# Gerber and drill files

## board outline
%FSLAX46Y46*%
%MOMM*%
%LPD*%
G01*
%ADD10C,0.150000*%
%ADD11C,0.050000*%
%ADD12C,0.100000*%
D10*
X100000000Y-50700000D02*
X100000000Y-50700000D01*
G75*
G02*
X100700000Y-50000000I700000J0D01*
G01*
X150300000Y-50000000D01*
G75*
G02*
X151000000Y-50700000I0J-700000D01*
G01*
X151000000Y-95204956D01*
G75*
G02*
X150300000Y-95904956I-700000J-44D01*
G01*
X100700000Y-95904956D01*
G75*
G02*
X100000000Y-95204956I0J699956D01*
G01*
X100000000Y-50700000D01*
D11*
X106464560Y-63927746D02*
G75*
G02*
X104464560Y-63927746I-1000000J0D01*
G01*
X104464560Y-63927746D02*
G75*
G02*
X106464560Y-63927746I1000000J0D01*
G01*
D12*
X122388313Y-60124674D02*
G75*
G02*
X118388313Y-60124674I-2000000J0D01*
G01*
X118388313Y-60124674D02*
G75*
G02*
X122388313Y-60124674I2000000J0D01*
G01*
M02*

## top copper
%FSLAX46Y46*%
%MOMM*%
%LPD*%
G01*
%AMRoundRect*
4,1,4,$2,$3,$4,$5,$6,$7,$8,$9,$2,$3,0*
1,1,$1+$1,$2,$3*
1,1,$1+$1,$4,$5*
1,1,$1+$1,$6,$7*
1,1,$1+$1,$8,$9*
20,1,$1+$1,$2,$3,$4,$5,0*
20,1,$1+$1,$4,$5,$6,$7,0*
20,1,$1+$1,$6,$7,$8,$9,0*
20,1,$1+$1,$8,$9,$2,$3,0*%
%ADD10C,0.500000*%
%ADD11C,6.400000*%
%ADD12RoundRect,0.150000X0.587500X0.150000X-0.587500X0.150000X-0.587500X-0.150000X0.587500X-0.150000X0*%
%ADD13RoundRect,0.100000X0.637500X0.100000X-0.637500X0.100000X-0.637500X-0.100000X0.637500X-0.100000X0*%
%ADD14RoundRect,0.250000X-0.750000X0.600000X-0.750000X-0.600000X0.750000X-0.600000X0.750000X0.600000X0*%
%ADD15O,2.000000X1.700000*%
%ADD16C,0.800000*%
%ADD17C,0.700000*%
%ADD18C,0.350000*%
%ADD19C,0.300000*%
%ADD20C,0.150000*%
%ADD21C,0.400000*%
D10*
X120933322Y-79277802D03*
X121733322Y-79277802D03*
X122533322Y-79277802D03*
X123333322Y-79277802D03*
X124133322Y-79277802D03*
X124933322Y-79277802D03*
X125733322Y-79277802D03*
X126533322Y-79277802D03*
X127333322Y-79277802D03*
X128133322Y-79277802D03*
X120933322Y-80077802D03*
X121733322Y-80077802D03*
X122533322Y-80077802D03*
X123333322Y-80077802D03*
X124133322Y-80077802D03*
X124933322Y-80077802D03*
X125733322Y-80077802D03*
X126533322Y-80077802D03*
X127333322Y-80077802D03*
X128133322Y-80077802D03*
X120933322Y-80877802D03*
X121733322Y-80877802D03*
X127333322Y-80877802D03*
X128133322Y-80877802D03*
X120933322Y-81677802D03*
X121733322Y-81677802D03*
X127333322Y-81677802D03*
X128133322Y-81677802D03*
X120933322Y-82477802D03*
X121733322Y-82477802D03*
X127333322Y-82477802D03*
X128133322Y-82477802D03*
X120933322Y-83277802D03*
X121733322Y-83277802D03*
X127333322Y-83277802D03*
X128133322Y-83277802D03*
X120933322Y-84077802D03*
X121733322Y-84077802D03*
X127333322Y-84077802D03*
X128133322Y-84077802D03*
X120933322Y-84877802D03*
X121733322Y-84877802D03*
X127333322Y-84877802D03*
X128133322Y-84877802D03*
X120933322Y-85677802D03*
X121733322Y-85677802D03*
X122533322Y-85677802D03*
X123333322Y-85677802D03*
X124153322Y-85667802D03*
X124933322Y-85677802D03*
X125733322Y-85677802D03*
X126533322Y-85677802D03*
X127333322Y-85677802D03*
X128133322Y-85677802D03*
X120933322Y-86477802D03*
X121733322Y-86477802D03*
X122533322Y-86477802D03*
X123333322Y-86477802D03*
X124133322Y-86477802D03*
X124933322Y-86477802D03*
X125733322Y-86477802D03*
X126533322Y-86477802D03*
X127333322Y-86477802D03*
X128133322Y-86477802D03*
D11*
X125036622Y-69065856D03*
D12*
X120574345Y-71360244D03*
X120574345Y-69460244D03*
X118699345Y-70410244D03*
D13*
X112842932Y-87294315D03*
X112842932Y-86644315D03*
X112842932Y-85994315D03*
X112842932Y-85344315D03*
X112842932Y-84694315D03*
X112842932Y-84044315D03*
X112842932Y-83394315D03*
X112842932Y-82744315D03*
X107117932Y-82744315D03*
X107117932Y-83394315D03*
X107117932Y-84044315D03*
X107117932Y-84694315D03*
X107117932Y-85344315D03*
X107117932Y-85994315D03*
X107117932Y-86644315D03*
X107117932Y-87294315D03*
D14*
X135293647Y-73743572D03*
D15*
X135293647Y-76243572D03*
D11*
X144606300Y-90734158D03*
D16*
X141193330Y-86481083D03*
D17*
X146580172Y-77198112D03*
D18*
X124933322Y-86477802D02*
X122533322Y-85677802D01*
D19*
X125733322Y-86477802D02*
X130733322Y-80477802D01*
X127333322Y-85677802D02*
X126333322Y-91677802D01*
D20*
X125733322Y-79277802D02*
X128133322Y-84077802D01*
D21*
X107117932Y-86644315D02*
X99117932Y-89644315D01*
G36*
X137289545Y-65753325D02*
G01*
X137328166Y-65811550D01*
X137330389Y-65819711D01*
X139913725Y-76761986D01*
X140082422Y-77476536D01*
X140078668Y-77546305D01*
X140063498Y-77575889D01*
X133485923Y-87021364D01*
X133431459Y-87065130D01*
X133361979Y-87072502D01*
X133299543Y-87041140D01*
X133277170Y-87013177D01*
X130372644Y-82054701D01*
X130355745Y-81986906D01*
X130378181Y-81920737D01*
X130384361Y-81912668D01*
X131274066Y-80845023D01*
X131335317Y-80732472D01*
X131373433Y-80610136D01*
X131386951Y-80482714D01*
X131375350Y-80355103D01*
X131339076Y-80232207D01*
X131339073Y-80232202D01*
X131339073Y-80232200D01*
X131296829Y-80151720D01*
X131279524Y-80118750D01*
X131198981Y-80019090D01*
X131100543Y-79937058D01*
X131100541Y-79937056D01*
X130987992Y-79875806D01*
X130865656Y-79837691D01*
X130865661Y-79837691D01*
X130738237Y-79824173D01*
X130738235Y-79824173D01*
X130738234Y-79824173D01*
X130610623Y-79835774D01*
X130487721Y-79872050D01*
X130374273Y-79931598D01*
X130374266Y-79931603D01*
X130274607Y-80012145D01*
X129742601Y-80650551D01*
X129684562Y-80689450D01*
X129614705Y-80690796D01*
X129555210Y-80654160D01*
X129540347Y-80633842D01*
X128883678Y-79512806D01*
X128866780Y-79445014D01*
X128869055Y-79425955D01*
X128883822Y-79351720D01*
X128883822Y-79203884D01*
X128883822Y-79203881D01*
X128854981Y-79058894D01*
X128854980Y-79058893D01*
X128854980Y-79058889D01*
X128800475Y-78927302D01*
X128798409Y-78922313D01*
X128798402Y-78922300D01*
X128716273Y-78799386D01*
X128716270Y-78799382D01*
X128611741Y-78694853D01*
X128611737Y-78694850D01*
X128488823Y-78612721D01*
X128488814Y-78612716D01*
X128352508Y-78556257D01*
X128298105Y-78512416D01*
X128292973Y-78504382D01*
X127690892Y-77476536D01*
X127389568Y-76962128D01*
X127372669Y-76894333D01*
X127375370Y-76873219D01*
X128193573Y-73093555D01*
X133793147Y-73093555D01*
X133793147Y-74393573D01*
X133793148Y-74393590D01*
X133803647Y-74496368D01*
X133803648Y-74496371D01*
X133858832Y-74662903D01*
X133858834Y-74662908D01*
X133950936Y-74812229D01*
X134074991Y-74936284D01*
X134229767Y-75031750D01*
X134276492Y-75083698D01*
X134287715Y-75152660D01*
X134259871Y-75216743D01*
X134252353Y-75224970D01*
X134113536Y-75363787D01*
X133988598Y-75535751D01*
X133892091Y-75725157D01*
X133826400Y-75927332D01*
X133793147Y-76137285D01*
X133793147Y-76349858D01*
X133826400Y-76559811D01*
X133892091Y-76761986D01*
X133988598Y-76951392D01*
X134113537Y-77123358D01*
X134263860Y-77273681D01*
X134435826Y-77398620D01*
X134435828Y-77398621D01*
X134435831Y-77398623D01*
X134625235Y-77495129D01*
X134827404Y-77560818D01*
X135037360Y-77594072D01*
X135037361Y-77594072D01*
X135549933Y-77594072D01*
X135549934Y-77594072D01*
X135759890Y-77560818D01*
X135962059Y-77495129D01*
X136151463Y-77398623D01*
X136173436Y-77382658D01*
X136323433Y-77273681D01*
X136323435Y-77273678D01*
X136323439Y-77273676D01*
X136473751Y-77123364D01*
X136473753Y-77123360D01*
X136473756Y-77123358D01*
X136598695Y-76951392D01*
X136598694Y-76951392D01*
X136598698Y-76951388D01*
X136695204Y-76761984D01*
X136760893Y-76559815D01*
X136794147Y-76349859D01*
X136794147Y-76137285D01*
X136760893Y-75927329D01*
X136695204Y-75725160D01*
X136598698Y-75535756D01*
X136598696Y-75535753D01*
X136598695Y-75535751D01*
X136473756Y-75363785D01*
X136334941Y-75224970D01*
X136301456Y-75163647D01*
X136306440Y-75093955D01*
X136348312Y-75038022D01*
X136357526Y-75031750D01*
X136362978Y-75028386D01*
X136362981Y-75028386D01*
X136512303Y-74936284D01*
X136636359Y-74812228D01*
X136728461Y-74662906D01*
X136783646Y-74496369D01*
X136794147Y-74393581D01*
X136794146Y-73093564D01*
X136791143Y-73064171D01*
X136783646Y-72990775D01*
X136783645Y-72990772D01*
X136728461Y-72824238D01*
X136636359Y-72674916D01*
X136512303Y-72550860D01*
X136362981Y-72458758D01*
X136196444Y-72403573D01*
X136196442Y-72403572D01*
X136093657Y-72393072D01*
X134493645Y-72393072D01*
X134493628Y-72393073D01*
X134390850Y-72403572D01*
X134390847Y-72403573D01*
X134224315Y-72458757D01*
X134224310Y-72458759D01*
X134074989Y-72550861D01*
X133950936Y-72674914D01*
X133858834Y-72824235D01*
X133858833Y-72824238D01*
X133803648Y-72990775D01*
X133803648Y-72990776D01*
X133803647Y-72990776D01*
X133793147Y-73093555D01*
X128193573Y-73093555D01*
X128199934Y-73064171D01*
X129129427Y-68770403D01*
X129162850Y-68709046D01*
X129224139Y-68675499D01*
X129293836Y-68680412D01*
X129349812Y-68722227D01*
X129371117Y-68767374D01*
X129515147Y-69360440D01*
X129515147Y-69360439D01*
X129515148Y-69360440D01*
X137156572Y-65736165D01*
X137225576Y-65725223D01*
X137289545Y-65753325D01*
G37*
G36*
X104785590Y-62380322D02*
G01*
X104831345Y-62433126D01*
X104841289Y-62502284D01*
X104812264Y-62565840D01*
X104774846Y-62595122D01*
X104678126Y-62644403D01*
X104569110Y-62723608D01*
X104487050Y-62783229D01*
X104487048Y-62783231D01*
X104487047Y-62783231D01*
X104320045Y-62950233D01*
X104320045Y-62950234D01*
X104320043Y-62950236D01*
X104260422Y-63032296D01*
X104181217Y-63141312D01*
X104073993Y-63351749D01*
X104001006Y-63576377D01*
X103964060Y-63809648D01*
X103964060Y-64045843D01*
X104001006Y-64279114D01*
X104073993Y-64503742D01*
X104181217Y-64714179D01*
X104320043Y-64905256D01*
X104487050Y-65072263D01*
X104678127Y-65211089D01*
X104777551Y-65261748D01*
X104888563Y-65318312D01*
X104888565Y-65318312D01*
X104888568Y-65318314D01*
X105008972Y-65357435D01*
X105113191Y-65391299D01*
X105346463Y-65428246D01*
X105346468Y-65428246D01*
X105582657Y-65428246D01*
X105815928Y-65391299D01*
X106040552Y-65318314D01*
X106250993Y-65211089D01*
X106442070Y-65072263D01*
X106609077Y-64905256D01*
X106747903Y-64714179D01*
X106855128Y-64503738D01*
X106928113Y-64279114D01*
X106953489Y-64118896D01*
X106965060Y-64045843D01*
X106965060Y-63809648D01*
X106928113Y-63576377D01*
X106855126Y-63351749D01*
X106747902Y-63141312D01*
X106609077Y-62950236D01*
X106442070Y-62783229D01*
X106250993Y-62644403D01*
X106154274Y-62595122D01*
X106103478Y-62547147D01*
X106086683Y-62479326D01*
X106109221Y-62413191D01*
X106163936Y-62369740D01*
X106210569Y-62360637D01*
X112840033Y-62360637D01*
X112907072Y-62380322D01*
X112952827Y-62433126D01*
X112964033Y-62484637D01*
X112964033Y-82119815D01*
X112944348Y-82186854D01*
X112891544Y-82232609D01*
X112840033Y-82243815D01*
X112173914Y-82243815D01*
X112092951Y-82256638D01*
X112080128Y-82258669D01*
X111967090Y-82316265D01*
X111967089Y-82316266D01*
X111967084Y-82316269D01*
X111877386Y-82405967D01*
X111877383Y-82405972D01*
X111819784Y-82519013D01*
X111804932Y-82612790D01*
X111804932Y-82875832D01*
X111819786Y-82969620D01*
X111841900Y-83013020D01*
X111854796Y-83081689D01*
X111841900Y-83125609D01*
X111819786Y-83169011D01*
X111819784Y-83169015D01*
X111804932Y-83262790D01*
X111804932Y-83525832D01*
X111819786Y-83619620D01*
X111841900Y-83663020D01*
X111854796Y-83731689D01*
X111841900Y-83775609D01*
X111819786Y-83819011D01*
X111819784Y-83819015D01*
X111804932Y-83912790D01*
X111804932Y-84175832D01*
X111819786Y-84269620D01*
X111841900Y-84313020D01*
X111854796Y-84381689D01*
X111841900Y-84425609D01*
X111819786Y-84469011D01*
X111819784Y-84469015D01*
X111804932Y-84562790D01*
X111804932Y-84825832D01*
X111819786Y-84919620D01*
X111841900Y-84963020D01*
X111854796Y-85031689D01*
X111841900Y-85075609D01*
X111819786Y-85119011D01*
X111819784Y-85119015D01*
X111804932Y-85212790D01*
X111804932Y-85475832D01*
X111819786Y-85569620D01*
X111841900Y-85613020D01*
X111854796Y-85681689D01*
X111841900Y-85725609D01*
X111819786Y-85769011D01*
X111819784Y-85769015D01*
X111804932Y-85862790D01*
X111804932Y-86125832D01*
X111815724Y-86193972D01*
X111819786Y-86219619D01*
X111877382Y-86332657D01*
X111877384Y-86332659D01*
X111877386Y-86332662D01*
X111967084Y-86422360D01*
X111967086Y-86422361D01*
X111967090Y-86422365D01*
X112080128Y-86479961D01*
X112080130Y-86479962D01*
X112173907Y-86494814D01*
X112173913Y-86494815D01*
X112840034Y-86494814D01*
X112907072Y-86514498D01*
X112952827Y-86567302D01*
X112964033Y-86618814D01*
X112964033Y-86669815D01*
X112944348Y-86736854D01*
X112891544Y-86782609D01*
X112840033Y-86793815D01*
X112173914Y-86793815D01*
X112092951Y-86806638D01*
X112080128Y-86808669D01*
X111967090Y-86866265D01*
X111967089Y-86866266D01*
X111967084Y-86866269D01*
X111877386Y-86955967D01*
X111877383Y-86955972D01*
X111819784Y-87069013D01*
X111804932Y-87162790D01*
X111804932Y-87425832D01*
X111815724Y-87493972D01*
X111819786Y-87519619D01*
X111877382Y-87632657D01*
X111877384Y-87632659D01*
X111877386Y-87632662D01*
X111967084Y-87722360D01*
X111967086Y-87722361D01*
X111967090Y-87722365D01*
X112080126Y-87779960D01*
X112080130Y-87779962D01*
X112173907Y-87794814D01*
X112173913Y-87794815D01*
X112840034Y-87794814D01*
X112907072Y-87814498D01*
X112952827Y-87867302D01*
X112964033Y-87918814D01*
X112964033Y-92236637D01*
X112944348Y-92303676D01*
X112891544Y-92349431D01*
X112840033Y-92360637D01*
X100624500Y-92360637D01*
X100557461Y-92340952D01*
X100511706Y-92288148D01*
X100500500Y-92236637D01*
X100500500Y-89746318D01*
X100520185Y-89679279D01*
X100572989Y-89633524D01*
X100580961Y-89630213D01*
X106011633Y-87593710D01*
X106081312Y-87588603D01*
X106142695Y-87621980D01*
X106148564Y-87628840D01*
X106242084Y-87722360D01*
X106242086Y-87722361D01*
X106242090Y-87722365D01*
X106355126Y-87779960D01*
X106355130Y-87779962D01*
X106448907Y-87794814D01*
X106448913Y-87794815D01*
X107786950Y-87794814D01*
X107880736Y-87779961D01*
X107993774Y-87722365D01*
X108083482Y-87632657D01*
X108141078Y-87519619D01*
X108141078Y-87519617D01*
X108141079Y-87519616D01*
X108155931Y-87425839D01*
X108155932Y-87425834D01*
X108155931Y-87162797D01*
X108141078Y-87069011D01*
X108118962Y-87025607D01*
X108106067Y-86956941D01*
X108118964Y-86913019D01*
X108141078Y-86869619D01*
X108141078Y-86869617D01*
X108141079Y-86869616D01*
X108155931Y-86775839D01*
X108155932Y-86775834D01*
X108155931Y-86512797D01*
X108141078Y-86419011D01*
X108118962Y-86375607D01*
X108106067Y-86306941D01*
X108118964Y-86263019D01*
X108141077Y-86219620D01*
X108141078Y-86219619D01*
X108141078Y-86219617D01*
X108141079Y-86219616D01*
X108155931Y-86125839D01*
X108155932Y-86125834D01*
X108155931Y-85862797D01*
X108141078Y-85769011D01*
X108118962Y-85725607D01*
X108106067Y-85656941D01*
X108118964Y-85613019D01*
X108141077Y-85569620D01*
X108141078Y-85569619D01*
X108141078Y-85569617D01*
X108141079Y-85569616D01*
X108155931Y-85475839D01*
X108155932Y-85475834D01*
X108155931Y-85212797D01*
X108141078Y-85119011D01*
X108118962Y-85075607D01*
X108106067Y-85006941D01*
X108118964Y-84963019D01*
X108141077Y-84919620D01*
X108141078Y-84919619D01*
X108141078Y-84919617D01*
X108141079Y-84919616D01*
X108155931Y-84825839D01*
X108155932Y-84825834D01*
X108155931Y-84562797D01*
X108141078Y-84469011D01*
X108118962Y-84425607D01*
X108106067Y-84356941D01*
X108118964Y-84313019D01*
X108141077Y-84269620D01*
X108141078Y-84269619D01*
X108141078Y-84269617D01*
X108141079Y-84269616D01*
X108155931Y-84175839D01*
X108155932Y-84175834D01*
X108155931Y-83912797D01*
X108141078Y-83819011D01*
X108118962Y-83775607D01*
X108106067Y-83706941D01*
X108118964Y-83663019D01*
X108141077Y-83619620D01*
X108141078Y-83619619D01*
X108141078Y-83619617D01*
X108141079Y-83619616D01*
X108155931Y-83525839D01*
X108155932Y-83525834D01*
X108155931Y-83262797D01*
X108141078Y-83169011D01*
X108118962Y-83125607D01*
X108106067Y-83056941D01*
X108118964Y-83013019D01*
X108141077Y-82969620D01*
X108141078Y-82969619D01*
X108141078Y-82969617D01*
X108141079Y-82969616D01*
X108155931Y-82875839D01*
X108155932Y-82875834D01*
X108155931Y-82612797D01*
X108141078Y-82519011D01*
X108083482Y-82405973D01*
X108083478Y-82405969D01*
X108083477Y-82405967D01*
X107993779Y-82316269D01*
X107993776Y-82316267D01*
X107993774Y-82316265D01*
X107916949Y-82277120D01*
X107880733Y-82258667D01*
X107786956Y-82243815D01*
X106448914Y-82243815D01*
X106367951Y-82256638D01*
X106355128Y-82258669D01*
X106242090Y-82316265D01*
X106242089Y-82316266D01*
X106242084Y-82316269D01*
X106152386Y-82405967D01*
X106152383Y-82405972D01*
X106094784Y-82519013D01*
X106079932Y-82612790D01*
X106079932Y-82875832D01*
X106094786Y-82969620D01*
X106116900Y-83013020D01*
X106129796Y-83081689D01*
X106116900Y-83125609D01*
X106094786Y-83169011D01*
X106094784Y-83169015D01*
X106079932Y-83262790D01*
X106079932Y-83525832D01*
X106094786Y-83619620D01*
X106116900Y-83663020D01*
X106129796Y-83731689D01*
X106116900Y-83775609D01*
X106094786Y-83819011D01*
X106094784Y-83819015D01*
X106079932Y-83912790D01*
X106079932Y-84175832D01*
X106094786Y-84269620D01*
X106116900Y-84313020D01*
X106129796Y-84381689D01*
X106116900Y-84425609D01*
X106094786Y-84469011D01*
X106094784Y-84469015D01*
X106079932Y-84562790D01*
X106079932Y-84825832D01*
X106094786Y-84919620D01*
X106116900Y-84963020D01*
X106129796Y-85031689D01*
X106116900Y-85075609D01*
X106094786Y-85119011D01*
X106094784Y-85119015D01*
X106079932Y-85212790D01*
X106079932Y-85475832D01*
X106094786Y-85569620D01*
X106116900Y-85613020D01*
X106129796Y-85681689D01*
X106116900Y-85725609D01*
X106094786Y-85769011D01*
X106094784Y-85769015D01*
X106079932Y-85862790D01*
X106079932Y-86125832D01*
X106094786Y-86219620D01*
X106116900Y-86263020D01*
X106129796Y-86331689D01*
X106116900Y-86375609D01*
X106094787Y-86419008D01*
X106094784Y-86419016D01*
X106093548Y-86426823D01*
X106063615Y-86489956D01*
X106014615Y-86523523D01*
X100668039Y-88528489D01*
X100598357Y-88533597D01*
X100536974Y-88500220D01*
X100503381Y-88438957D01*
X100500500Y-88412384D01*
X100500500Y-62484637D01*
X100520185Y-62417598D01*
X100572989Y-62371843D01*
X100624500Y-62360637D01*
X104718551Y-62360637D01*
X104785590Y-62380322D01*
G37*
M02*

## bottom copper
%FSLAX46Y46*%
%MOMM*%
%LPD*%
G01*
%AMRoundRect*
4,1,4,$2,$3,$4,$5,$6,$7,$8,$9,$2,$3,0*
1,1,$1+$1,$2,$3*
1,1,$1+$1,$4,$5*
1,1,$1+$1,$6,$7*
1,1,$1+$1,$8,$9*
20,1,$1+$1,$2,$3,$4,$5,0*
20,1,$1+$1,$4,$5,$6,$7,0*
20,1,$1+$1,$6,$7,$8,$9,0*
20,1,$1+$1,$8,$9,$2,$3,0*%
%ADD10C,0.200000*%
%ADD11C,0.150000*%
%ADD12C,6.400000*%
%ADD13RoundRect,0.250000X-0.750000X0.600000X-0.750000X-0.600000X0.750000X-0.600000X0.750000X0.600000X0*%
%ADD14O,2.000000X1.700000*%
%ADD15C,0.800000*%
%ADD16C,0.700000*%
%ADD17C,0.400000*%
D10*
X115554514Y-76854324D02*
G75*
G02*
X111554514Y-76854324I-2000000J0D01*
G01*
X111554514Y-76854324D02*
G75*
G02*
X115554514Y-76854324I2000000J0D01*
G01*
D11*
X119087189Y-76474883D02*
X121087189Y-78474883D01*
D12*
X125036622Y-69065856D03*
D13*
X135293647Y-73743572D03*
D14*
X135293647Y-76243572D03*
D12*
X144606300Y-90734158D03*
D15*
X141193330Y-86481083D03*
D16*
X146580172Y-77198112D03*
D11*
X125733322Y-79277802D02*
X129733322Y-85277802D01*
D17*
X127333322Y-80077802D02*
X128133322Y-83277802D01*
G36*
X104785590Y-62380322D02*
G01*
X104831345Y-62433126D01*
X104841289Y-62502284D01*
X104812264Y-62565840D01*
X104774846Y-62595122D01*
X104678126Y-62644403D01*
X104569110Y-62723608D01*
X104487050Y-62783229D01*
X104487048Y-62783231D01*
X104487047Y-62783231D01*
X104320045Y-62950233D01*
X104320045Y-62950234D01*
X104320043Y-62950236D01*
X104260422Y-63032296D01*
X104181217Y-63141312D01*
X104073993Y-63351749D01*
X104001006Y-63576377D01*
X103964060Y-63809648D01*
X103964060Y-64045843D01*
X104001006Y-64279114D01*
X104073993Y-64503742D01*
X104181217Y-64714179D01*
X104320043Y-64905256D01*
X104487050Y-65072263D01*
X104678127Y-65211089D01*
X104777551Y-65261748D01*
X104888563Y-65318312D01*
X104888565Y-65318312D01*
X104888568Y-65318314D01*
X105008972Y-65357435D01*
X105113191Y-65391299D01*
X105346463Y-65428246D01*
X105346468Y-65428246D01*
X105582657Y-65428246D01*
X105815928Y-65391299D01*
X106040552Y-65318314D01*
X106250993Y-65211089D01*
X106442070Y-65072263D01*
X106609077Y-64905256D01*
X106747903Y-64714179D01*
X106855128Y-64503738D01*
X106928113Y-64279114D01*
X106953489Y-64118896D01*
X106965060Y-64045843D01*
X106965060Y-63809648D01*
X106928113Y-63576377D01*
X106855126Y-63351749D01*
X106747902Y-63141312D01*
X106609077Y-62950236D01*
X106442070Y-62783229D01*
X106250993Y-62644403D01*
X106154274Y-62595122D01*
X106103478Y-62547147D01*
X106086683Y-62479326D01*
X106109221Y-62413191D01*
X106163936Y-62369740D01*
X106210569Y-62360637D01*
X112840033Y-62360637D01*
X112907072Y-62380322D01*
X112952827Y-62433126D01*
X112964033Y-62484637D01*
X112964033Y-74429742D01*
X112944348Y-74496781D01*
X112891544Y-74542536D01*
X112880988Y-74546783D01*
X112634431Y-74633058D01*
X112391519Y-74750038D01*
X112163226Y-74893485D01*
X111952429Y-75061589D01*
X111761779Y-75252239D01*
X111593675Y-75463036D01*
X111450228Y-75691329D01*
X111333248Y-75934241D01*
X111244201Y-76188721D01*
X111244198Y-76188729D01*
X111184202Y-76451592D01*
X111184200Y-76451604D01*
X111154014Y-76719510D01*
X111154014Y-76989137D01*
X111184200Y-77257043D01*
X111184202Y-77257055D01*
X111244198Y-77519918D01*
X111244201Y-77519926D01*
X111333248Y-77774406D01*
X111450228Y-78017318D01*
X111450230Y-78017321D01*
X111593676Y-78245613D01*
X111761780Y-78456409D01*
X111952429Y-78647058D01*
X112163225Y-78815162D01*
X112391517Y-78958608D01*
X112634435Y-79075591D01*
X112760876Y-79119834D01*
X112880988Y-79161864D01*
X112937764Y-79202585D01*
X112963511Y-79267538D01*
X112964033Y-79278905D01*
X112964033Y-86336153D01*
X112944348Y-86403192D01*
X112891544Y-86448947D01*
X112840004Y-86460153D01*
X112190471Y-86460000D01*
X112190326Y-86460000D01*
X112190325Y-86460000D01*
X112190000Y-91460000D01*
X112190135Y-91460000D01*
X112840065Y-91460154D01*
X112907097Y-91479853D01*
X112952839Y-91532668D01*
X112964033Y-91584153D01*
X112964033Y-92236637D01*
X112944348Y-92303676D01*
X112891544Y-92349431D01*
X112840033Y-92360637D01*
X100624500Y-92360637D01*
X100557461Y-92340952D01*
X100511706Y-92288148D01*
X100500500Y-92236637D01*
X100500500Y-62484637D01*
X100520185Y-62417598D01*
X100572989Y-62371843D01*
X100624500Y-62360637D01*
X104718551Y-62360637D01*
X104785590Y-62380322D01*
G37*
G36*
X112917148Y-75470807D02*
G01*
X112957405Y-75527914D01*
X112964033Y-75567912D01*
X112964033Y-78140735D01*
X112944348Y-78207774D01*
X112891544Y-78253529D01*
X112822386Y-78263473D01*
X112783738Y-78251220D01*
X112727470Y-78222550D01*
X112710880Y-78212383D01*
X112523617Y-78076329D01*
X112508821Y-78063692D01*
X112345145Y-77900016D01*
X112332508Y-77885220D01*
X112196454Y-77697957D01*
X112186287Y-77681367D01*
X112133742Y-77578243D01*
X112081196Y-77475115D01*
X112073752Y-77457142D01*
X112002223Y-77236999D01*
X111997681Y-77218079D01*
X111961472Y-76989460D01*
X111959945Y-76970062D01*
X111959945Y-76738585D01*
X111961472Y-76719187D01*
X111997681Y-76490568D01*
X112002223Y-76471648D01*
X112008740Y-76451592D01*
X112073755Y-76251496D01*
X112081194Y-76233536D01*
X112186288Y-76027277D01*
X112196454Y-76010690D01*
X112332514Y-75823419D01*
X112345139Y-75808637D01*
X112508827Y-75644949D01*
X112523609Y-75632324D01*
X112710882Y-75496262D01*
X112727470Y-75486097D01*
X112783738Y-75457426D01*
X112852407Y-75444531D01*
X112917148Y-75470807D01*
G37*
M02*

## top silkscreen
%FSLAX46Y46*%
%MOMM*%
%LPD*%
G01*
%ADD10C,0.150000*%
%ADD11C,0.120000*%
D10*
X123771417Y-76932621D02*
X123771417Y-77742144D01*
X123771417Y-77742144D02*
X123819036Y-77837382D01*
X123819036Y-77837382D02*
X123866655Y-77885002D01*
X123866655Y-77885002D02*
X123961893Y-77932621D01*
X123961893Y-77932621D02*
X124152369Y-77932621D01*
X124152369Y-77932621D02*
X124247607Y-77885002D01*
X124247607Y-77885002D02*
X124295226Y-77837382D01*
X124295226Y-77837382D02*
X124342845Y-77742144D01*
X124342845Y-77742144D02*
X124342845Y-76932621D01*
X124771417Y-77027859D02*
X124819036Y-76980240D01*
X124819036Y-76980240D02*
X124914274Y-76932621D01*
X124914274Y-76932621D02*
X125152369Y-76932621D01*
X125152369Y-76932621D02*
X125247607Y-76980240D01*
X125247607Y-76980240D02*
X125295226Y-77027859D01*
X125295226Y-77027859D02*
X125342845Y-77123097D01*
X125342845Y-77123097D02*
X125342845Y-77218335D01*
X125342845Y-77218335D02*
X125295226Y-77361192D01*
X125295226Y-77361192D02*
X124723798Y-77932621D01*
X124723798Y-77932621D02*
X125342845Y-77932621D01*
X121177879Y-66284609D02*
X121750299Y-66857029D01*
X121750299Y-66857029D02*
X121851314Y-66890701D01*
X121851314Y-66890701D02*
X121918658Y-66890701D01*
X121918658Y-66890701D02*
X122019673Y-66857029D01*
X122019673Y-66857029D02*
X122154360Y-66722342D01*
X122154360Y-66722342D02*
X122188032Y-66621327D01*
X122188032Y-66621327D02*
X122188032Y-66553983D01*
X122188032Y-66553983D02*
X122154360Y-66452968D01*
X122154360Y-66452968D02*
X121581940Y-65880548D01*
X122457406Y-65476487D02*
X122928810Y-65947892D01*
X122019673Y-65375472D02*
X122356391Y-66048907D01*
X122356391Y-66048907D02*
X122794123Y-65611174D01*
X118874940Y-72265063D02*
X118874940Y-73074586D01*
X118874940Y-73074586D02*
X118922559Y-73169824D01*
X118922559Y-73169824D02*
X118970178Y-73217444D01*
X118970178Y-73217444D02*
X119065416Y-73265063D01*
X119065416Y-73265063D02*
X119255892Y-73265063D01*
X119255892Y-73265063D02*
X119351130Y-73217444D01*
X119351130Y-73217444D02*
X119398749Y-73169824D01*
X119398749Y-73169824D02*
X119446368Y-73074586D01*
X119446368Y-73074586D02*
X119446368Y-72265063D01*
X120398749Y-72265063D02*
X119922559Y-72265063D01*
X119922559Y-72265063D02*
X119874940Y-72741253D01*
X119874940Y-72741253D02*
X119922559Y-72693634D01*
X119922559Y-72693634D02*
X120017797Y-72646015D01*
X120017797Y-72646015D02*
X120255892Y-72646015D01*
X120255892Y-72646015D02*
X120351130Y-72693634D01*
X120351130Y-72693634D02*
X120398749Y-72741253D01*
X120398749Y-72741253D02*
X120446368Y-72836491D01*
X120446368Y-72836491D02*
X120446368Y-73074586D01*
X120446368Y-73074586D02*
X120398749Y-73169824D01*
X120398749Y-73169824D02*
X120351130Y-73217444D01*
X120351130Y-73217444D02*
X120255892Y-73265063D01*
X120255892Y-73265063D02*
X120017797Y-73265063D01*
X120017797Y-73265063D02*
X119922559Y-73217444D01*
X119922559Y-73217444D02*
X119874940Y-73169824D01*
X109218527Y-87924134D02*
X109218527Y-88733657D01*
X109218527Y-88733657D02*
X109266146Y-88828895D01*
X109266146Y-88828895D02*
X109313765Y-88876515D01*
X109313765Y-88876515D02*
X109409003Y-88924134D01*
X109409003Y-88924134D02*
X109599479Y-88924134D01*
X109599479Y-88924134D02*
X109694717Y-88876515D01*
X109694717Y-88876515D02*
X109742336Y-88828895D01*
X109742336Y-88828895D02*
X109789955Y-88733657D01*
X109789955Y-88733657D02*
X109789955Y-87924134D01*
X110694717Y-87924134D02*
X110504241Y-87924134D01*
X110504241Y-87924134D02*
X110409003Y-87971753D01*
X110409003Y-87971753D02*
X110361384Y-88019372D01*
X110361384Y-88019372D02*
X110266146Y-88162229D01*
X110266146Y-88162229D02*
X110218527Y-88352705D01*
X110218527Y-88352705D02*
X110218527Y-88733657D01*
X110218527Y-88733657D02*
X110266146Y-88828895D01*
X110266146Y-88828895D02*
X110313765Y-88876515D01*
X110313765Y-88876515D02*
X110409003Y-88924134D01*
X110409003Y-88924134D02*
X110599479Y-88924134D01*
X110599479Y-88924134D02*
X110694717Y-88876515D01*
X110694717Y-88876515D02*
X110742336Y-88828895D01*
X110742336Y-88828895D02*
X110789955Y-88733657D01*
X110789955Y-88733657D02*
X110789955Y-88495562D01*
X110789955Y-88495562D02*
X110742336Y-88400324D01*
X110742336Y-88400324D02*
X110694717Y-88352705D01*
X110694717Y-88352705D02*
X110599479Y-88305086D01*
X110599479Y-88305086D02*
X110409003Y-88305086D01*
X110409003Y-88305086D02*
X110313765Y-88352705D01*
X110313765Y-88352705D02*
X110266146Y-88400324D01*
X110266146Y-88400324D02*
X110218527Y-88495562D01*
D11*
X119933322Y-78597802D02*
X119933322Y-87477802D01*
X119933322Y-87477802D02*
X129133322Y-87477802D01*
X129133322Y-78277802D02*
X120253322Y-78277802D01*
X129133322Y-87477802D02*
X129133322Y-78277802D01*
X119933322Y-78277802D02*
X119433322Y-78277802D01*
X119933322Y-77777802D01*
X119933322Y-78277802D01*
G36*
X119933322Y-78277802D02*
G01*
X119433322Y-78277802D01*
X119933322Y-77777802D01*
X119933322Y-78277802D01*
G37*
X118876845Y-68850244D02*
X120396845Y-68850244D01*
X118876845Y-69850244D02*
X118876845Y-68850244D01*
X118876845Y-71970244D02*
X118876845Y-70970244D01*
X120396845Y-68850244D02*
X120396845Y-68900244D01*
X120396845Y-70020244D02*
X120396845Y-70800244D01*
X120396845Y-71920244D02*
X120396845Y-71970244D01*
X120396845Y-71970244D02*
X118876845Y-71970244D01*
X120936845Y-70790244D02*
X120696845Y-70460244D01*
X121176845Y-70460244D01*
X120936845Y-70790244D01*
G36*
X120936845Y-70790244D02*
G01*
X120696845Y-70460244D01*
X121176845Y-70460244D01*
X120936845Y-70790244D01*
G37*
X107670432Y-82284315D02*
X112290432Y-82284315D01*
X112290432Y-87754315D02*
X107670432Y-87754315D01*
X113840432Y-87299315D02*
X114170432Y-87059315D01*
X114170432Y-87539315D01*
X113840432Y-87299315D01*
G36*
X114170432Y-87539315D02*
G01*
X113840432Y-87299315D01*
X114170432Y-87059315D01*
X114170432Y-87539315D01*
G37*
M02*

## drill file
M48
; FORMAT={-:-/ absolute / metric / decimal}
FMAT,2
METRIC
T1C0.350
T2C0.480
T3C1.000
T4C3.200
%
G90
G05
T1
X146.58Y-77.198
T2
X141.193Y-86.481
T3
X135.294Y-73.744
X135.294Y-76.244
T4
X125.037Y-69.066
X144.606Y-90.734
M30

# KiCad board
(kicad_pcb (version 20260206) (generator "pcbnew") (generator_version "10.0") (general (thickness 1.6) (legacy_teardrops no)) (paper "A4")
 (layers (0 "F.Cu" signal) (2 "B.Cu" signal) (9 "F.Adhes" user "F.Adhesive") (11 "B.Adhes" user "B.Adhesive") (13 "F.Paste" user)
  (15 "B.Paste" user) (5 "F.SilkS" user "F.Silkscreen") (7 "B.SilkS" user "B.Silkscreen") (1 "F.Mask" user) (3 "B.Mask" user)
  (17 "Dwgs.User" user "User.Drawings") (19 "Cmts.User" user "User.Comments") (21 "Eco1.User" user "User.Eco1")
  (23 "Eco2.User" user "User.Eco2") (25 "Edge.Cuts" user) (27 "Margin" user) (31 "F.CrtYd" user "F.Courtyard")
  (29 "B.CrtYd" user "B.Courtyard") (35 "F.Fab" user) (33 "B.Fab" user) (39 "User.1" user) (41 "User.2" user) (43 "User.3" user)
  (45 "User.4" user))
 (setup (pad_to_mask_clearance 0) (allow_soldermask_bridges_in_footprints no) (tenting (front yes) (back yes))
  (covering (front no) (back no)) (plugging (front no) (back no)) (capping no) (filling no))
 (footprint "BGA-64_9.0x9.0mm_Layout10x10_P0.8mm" (layer "F.Cu") (at 124.533322 82.877802)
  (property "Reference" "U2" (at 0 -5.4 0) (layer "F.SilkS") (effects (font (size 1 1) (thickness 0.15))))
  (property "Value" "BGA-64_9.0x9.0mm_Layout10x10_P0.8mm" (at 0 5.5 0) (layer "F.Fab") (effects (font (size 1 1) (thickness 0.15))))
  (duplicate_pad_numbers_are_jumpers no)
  (fp_line (start -4.6 -4.28) (end -4.6 4.6) (stroke (width 0.12) (type solid)) (layer "F.SilkS"))
  (fp_line (start -4.6 4.6) (end 4.6 4.6) (stroke (width 0.12) (type solid)) (layer "F.SilkS"))
  (fp_line (start 4.6 -4.6) (end -4.28 -4.6) (stroke (width 0.12) (type solid)) (layer "F.SilkS"))
  (fp_line (start 4.6 4.6) (end 4.6 -4.6) (stroke (width 0.12) (type solid)) (layer "F.SilkS"))
  (fp_poly
   (pts (xy -4.6 -4.6) (xy -5.1 -4.6) (xy -4.6 -5.1) (xy -4.6 -4.6)) (stroke (width 0.12) (type solid)) (fill yes) (layer "F.SilkS"))
  (pad "A1" smd circle (at -3.6 -3.6) (size 0.5 0.5) (layers "F.Cu" "F.Mask" "F.Paste") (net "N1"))
  (pad "A2" smd circle (at -2.8 -3.6) (size 0.5 0.5) (layers "F.Cu" "F.Mask" "F.Paste"))
  (pad "A3" smd circle (at -2 -3.6) (size 0.5 0.5) (layers "F.Cu" "F.Mask" "F.Paste") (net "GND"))
  (pad "A4" smd circle (at -1.2 -3.6) (size 0.5 0.5) (layers "F.Cu" "F.Mask" "F.Paste") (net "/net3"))
  (pad "A5" smd circle (at -0.4 -3.6) (size 0.5 0.5) (layers "F.Cu" "F.Mask" "F.Paste") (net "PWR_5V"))
  (pad "A6" smd circle (at 0.4 -3.6) (size 0.5 0.5) (layers "F.Cu" "F.Mask" "F.Paste"))
  (pad "A7" smd circle (at 1.2 -3.6) (size 0.5 0.5) (layers "F.Cu" "F.Mask" "F.Paste") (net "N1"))
  (pad "A8" smd circle (at 2 -3.6) (size 0.5 0.5) (layers "F.Cu" "F.Mask" "F.Paste") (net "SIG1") (clearance 0.1))
  (pad "A9" smd circle (at 2.8 -3.6) (size 0.5 0.5) (layers "F.Cu" "F.Mask" "F.Paste") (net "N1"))
  (pad "A10" smd circle (at 3.6 -3.6) (size 0.5 0.5) (layers "F.Cu" "F.Mask" "F.Paste") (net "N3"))
  (pad "B1" smd circle (at -3.6 -2.8) (size 0.5 0.5) (layers "F.Cu" "F.Mask" "F.Paste"))
  (pad "B2" smd circle (at -2.8 -2.8) (size 0.5 0.5) (layers "F.Cu" "F.Mask" "F.Paste") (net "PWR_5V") (clearance 0.35))
  (pad "B3" smd circle (at -2 -2.8) (size 0.5 0.5) (layers "F.Cu" "F.Mask" "F.Paste") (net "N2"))
  (pad "B4" smd circle (at -1.2 -2.8) (size 0.5 0.5) (layers "F.Cu" "F.Mask" "F.Paste"))
  (pad "B5" smd circle (at -0.4 -2.8) (size 0.5 0.5) (layers "F.Cu" "F.Mask" "F.Paste"))
  (pad "B6" smd circle (at 0.4 -2.8) (size 0.5 0.5) (layers "F.Cu" "F.Mask" "F.Paste"))
  (pad "B7" smd circle (at 1.2 -2.8) (size 0.5 0.5) (layers "F.Cu" "F.Mask" "F.Paste") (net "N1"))
  (pad "B8" smd circle (at 2 -2.8) (size 0.5 0.5) (layers "F.Cu" "F.Mask" "F.Paste"))
  (pad "B9" smd circle (at 2.8 -2.8) (size 0.5 0.5) (layers "F.Cu" "F.Mask" "F.Paste") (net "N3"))
  (pad "B10" smd circle (at 3.6 -2.8) (size 0.5 0.5) (layers "F.Cu" "F.Mask" "F.Paste") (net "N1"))
  (pad "C1" smd circle (at -3.6 -2) (size 0.5 0.5) (layers "F.Cu" "F.Mask" "F.Paste"))
  (pad "C2" smd circle (at -2.8 -2) (size 0.5 0.5) (layers "F.Cu" "F.Mask" "F.Paste") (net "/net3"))
  (pad "C9" smd circle (at 2.8 -2) (size 0.5 0.5) (layers "F.Cu" "F.Mask" "F.Paste"))
  (pad "C10" smd circle (at 3.6 -2) (size 0.5 0.5) (layers "F.Cu" "F.Mask" "F.Paste") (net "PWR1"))
  (pad "D1" smd circle (at -3.6 -1.2) (size 0.5 0.5) (layers "F.Cu" "F.Mask" "F.Paste") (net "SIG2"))
  (pad "D2" smd circle (at -2.8 -1.2) (size 0.5 0.5) (layers "F.Cu" "F.Mask" "F.Paste") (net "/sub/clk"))
  (pad "D9" smd circle (at 2.8 -1.2) (size 0.5 0.5) (layers "F.Cu" "F.Mask" "F.Paste") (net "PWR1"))
  (pad "D10" smd circle (at 3.6 -1.2) (size 0.5 0.5) (layers "F.Cu" "F.Mask" "F.Paste") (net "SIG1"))
  (pad "E1" smd circle (at -3.6 -0.4) (size 0.5 0.5) (layers "F.Cu" "F.Mask" "F.Paste") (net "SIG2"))
  (pad "E2" smd circle (at -2.8 -0.4) (size 0.5 0.5) (layers "F.Cu" "F.Mask" "F.Paste"))
  (pad "E9" smd circle (at 2.8 -0.4) (size 0.5 0.5) (layers "F.Cu" "F.Mask" "F.Paste") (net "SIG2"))
  (pad "E10" smd circle (at 3.6 -0.4) (size 0.5 0.5) (layers "F.Cu" "F.Mask" "F.Paste") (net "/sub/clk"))
  (pad "F1" smd circle (at -3.6 0.4) (size 0.5 0.5) (layers "F.Cu" "F.Mask" "F.Paste") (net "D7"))
  (pad "F2" smd circle (at -2.8 0.4) (size 0.5 0.5) (layers "F.Cu" "F.Mask" "F.Paste") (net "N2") (clearance 0.1))
  (pad "F9" smd circle (at 2.8 0.4) (size 0.5 0.5) (layers "F.Cu" "F.Mask" "F.Paste"))
  (pad "F10" smd circle (at 3.6 0.4) (size 0.5 0.5) (layers "F.Cu" "F.Mask" "F.Paste"))
  (pad "G1" smd circle (at -3.6 1.2) (size 0.5 0.5) (layers "F.Cu" "F.Mask" "F.Paste"))
  (pad "G2" smd circle (at -2.8 1.2) (size 0.5 0.5) (layers "F.Cu" "F.Mask" "F.Paste") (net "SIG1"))
  (pad "G9" smd circle (at 2.8 1.2) (size 0.5 0.5) (layers "F.Cu" "F.Mask" "F.Paste"))
  (pad "G10" smd circle (at 3.6 1.2) (size 0.5 0.5) (layers "F.Cu" "F.Mask" "F.Paste"))
  (pad "H1" smd circle (at -3.6 2) (size 0.5 0.5) (layers "F.Cu" "F.Mask" "F.Paste") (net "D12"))
  (pad "H2" smd circle (at -2.8 2) (size 0.5 0.5) (layers "F.Cu" "F.Mask" "F.Paste") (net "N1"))
  (pad "H9" smd circle (at 2.8 2) (size 0.5 0.5) (layers "F.Cu" "F.Mask" "F.Paste") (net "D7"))
  (pad "H10" smd circle (at 3.6 2) (size 0.5 0.5) (layers "F.Cu" "F.Mask" "F.Paste") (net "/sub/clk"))
  (pad "J1" smd circle (at -3.6 2.8) (size 0.5 0.5) (layers "F.Cu" "F.Mask" "F.Paste") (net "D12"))
  (pad "J2" smd circle (at -2.8 2.8) (size 0.5 0.5) (layers "F.Cu" "F.Mask" "F.Paste") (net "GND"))
  (pad "J3" smd circle (at -2 2.8) (size 0.5 0.5) (layers "F.Cu" "F.Mask" "F.Paste") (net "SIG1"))
  (pad "J4" smd circle (at -1.2 2.8) (size 0.5 0.5) (layers "F.Cu" "F.Mask" "F.Paste"))
  (pad "J5" smd circle (at -0.38 2.79) (size 0.5 0.5) (layers "F.Cu" "F.Mask" "F.Paste") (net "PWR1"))
  (pad "J6" smd circle (at 0.4 2.8) (size 0.5 0.5) (layers "F.Cu" "F.Mask" "F.Paste") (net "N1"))
  (pad "J7" smd circle (at 1.2 2.8) (size 0.5 0.5) (layers "F.Cu" "F.Mask" "F.Paste") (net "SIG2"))
  (pad "J8" smd circle (at 2 2.8) (size 0.5 0.5) (layers "F.Cu" "F.Mask" "F.Paste") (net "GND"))
  (pad "J9" smd circle (at 2.8 2.8) (size 0.5 0.5) (layers "F.Cu" "F.Mask" "F.Paste"))
  (pad "J10" smd circle (at 3.6 2.8) (size 0.5 0.5) (layers "F.Cu" "F.Mask" "F.Paste"))
  (pad "K1" smd circle (at -3.6 3.6) (size 0.5 0.5) (layers "F.Cu" "F.Mask" "F.Paste") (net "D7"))
  (pad "K2" smd circle (at -2.8 3.6) (size 0.5 0.5) (layers "F.Cu" "F.Mask" "F.Paste") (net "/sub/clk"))
  (pad "K3" smd circle (at -2 3.6) (size 0.5 0.5) (layers "F.Cu" "F.Mask" "F.Paste") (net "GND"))
  (pad "K4" smd circle (at -1.2 3.6) (size 0.5 0.5) (layers "F.Cu" "F.Mask" "F.Paste") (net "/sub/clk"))
  (pad "K5" smd circle (at -0.4 3.6) (size 0.5 0.5) (layers "F.Cu" "F.Mask" "F.Paste") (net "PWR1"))
  (pad "K6" smd circle (at 0.4 3.6) (size 0.5 0.5) (layers "F.Cu" "F.Mask" "F.Paste") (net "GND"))
  (pad "K7" smd circle (at 1.2 3.6) (size 0.5 0.5) (layers "F.Cu" "F.Mask" "F.Paste") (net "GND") (clearance 0.35))
  (pad "K8" smd circle (at 2 3.6) (size 0.5 0.5) (layers "F.Cu" "F.Mask" "F.Paste") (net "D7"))
  (pad "K9" smd circle (at 2.8 3.6) (size 0.5 0.5) (layers "F.Cu" "F.Mask" "F.Paste") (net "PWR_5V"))
  (pad "K10" smd circle (at 3.6 3.6) (size 0.5 0.5) (layers "F.Cu" "F.Mask" "F.Paste") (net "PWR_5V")))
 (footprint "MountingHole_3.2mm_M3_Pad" (layer "F.Cu") (at 125.036622 69.065856 45)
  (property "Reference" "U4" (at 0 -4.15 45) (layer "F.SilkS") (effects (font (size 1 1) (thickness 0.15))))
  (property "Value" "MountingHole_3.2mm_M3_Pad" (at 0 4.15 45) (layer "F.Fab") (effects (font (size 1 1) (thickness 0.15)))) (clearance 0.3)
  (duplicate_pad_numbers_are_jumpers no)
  (pad "1" thru_hole circle (at 0 0 45) (size 6.4 6.4) (drill 3.2) (layers "*.Cu" "*.Mask") (remove_unused_layers no) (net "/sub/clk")
   (zone_connect 2)))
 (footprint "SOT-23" (layer "F.Cu") (at 119.636845 70.410244 180)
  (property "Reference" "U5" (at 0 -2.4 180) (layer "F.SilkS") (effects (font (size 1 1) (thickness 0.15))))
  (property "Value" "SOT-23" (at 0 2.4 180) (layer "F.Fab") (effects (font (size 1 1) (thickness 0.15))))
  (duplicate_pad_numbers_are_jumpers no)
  (fp_line (start 0.76 1.56) (end -0.76 1.56) (stroke (width 0.12) (type solid)) (layer "F.SilkS"))
  (fp_line (start 0.76 0.56) (end 0.76 1.56) (stroke (width 0.12) (type solid)) (layer "F.SilkS"))
  (fp_line (start 0.76 -1.56) (end 0.76 -0.56) (stroke (width 0.12) (type solid)) (layer "F.SilkS"))
  (fp_line (start -0.76 1.56) (end -0.76 1.51) (stroke (width 0.12) (type solid)) (layer "F.SilkS"))
  (fp_line (start -0.76 0.39) (end -0.76 -0.39) (stroke (width 0.12) (type solid)) (layer "F.SilkS"))
  (fp_line (start -0.76 -1.51) (end -0.76 -1.56) (stroke (width 0.12) (type solid)) (layer "F.SilkS"))
  (fp_line (start -0.76 -1.56) (end 0.76 -1.56) (stroke (width 0.12) (type solid)) (layer "F.SilkS"))
  (fp_poly (pts (xy -1.3 -0.38) (xy -1.06 -0.05) (xy -1.54 -0.05)) (stroke (width 0.12) (type solid)) (fill yes) (layer "F.SilkS"))
  (pad "1" smd roundrect (at -0.9375 -0.95 180) (size 1.475 0.6) (layers "F.Cu" "F.Mask" "F.Paste") (roundrect_rratio 0.25))
  (pad "2" smd roundrect (at -0.9375 0.95 180) (size 1.475 0.6) (layers "F.Cu" "F.Mask" "F.Paste") (roundrect_rratio 0.25) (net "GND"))
  (pad "3" smd roundrect (at 0.9375 0 180) (size 1.475 0.6) (layers "F.Cu" "F.Mask" "F.Paste") (roundrect_rratio 0.25) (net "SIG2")))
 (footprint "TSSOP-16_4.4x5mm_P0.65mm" (layer "F.Cu") (at 109.980432 85.019315 180)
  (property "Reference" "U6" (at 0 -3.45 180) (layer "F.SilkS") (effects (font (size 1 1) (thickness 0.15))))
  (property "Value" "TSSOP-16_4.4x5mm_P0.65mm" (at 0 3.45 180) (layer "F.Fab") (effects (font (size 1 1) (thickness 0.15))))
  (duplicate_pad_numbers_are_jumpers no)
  (fp_line (start 2.31 2.735) (end -2.31 2.735) (stroke (width 0.12) (type solid)) (layer "F.SilkS"))
  (fp_line (start -2.31 -2.735) (end 2.31 -2.735) (stroke (width 0.12) (type solid)) (layer "F.SilkS"))
  (fp_poly (pts (xy -3.86 -2.28) (xy -4.19 -2.04) (xy -4.19 -2.52)) (stroke (width 0.12) (type solid)) (fill yes) (layer "F.SilkS"))
  (pad "1" smd roundrect (at -2.8625 -2.275 180) (size 1.475 0.4) (layers "F.Cu" "F.Mask" "F.Paste") (roundrect_rratio 0.25) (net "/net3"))
  (pad "2" smd roundrect (at -2.8625 -1.625 180) (size 1.475 0.4) (layers "F.Cu" "F.Mask" "F.Paste") (roundrect_rratio 0.25) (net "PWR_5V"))
  (pad "3" smd roundrect (at -2.8625 -0.975 180) (size 1.475 0.4) (layers "F.Cu" "F.Mask" "F.Paste") (roundrect_rratio 0.25) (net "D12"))
  (pad "4" smd roundrect (at -2.8625 -0.325 180) (size 1.475 0.4) (layers "F.Cu" "F.Mask" "F.Paste") (roundrect_rratio 0.25) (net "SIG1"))
  (pad "5" smd roundrect (at -2.8625 0.325 180) (size 1.475 0.4) (layers "F.Cu" "F.Mask" "F.Paste") (roundrect_rratio 0.25) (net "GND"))
  (pad "6" smd roundrect (at -2.8625 0.975 180) (size 1.475 0.4) (layers "F.Cu" "F.Mask" "F.Paste") (roundrect_rratio 0.25))
  (pad "7" smd roundrect (at -2.8625 1.625 180) (size 1.475 0.4) (layers "F.Cu" "F.Mask" "F.Paste") (roundrect_rratio 0.25) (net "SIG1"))
  (pad "8" smd roundrect (at -2.8625 2.275 180) (size 1.475 0.4) (layers "F.Cu" "F.Mask" "F.Paste") (roundrect_rratio 0.25) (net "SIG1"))
  (pad "9" smd roundrect (at 2.8625 2.275 180) (size 1.475 0.4) (layers "F.Cu" "F.Mask" "F.Paste") (roundrect_rratio 0.25) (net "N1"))
  (pad "10" smd roundrect (at 2.8625 1.625 180) (size 1.475 0.4) (layers "F.Cu" "F.Mask" "F.Paste") (roundrect_rratio 0.25) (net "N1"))
  (pad "11" smd roundrect (at 2.8625 0.975 180) (size 1.475 0.4) (layers "F.Cu" "F.Mask" "F.Paste") (roundrect_rratio 0.25) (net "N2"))
  (pad "12" smd roundrect (at 2.8625 0.325 180) (size 1.475 0.4) (layers "F.Cu" "F.Mask" "F.Paste") (roundrect_rratio 0.25) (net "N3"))
  (pad "13" smd roundrect (at 2.8625 -0.325 180) (size 1.475 0.4) (layers "F.Cu" "F.Mask" "F.Paste") (roundrect_rratio 0.25) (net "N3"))
  (pad "14" smd roundrect (at 2.8625 -0.975 180) (size 1.475 0.4) (layers "F.Cu" "F.Mask" "F.Paste") (roundrect_rratio 0.25))
  (pad "15" smd roundrect (at 2.8625 -1.625 180) (size 1.475 0.4) (layers "F.Cu" "F.Mask" "F.Paste") (roundrect_rratio 0.25) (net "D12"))
  (pad "16" smd roundrect (at 2.8625 -2.275 180) (size 1.475 0.4) (layers "F.Cu" "F.Mask" "F.Paste") (roundrect_rratio 0.25) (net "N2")))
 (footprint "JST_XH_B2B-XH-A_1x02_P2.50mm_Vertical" (layer "B.Cu") (at 135.293647 73.743572 -90)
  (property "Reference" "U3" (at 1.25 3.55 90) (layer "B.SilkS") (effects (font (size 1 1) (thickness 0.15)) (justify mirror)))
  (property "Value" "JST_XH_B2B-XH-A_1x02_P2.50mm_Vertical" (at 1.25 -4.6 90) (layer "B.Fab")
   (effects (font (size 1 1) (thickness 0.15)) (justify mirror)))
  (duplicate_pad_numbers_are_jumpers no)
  (pad "1" thru_hole roundrect (at 0 0 270) (size 1.7 2) (drill 1) (layers "*.Cu" "*.Mask") (remove_unused_layers no)
   (roundrect_rratio 0.147059) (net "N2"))
  (pad "2" thru_hole oval (at 2.5 0 270) (size 1.7 2) (drill 1) (layers "*.Cu" "*.Mask") (remove_unused_layers no) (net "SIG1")))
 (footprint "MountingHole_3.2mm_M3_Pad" (layer "B.Cu") (at 144.6063 90.734158 -34.3)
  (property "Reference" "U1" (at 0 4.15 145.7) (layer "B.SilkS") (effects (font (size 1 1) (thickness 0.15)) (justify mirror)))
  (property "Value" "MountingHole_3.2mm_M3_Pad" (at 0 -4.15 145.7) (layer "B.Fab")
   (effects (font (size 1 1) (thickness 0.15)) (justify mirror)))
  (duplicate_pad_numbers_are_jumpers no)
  (pad "1" thru_hole circle (at 0 0 325.7) (size 6.4 6.4) (drill 3.2) (layers "*.Cu" "*.Mask") (remove_unused_layers no) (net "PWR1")
   (zone_connect 2)))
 (gr_circle (center 113.554514 76.854324) (end 115.554514 76.854324) (stroke (width 0.2) (type default)) (fill no) (layer "B.Cu")
  (net "/net3"))
 (gr_line (start 119.087189 76.474883) (end 121.087189 78.474883) (stroke (width 0.15) (type default)) (layer "B.Cu") (net "N2"))
 (gr_rect (start 100 50) (end 151 95.904956) (radius 0.7) (stroke (width 0.15) (type default)) (fill no) (layer "Edge.Cuts"))
 (gr_circle (center 105.46456 63.927746) (end 106.46456 63.927746) (stroke (width 0.05) (type default)) (fill no) (layer "Edge.Cuts"))
 (gr_circle (center 120.388313 60.124674) (end 122.388313 60.124674) (stroke (width 0.1) (type default)) (fill no) (layer "Edge.Cuts"))
 (segment (start 124.933322 86.477802) (end 122.533322 85.677802) (width 0.35) (layer "F.Cu") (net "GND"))
 (segment (start 125.733322 86.477802) (end 130.733322 80.477802) (width 0.3) (layer "F.Cu") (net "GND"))
 (segment (start 127.333322 85.677802) (end 126.333322 91.677802) (width 0.3) (layer "F.Cu") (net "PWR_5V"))
 (via (at 141.19333 86.481083) (size 0.8) (drill 0.48) (layers "F.Cu" "B.Cu") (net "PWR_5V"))
 (segment (start 125.733322 79.277802) (end 129.733322 85.277802) (width 0.15) (layer "B.Cu") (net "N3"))
 (segment (start 127.333322 80.077802) (end 128.133322 83.277802) (width 0.4) (layer "B.Cu") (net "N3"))
 (segment (start 125.733322 79.277802) (end 128.133322 84.077802) (width 0.15) (layer "F.Cu") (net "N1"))
 (segment (start 107.117932 86.644315) (end 99.117932 89.644315) (width 0.4) (layer "F.Cu") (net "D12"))
 (via (at 146.580172 77.198112) (size 0.7) (drill 0.35) (layers "F.Cu" "B.Cu") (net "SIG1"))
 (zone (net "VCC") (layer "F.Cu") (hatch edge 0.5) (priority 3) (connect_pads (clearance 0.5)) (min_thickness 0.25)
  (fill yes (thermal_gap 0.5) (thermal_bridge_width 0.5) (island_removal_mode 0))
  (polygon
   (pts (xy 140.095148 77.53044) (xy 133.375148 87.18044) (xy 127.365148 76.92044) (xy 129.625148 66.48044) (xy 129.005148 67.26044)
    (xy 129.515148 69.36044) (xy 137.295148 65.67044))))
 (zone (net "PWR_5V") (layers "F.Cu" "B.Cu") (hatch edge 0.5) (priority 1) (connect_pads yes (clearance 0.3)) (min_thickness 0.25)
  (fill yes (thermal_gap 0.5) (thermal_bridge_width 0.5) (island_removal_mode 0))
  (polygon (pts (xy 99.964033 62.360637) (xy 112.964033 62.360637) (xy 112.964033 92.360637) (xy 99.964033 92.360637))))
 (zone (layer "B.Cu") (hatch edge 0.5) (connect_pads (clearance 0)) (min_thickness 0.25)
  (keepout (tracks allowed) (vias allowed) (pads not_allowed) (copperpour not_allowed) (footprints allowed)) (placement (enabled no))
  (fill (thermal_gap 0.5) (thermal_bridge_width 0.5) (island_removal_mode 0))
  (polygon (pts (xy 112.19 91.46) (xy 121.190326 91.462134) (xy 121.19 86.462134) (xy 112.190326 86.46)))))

